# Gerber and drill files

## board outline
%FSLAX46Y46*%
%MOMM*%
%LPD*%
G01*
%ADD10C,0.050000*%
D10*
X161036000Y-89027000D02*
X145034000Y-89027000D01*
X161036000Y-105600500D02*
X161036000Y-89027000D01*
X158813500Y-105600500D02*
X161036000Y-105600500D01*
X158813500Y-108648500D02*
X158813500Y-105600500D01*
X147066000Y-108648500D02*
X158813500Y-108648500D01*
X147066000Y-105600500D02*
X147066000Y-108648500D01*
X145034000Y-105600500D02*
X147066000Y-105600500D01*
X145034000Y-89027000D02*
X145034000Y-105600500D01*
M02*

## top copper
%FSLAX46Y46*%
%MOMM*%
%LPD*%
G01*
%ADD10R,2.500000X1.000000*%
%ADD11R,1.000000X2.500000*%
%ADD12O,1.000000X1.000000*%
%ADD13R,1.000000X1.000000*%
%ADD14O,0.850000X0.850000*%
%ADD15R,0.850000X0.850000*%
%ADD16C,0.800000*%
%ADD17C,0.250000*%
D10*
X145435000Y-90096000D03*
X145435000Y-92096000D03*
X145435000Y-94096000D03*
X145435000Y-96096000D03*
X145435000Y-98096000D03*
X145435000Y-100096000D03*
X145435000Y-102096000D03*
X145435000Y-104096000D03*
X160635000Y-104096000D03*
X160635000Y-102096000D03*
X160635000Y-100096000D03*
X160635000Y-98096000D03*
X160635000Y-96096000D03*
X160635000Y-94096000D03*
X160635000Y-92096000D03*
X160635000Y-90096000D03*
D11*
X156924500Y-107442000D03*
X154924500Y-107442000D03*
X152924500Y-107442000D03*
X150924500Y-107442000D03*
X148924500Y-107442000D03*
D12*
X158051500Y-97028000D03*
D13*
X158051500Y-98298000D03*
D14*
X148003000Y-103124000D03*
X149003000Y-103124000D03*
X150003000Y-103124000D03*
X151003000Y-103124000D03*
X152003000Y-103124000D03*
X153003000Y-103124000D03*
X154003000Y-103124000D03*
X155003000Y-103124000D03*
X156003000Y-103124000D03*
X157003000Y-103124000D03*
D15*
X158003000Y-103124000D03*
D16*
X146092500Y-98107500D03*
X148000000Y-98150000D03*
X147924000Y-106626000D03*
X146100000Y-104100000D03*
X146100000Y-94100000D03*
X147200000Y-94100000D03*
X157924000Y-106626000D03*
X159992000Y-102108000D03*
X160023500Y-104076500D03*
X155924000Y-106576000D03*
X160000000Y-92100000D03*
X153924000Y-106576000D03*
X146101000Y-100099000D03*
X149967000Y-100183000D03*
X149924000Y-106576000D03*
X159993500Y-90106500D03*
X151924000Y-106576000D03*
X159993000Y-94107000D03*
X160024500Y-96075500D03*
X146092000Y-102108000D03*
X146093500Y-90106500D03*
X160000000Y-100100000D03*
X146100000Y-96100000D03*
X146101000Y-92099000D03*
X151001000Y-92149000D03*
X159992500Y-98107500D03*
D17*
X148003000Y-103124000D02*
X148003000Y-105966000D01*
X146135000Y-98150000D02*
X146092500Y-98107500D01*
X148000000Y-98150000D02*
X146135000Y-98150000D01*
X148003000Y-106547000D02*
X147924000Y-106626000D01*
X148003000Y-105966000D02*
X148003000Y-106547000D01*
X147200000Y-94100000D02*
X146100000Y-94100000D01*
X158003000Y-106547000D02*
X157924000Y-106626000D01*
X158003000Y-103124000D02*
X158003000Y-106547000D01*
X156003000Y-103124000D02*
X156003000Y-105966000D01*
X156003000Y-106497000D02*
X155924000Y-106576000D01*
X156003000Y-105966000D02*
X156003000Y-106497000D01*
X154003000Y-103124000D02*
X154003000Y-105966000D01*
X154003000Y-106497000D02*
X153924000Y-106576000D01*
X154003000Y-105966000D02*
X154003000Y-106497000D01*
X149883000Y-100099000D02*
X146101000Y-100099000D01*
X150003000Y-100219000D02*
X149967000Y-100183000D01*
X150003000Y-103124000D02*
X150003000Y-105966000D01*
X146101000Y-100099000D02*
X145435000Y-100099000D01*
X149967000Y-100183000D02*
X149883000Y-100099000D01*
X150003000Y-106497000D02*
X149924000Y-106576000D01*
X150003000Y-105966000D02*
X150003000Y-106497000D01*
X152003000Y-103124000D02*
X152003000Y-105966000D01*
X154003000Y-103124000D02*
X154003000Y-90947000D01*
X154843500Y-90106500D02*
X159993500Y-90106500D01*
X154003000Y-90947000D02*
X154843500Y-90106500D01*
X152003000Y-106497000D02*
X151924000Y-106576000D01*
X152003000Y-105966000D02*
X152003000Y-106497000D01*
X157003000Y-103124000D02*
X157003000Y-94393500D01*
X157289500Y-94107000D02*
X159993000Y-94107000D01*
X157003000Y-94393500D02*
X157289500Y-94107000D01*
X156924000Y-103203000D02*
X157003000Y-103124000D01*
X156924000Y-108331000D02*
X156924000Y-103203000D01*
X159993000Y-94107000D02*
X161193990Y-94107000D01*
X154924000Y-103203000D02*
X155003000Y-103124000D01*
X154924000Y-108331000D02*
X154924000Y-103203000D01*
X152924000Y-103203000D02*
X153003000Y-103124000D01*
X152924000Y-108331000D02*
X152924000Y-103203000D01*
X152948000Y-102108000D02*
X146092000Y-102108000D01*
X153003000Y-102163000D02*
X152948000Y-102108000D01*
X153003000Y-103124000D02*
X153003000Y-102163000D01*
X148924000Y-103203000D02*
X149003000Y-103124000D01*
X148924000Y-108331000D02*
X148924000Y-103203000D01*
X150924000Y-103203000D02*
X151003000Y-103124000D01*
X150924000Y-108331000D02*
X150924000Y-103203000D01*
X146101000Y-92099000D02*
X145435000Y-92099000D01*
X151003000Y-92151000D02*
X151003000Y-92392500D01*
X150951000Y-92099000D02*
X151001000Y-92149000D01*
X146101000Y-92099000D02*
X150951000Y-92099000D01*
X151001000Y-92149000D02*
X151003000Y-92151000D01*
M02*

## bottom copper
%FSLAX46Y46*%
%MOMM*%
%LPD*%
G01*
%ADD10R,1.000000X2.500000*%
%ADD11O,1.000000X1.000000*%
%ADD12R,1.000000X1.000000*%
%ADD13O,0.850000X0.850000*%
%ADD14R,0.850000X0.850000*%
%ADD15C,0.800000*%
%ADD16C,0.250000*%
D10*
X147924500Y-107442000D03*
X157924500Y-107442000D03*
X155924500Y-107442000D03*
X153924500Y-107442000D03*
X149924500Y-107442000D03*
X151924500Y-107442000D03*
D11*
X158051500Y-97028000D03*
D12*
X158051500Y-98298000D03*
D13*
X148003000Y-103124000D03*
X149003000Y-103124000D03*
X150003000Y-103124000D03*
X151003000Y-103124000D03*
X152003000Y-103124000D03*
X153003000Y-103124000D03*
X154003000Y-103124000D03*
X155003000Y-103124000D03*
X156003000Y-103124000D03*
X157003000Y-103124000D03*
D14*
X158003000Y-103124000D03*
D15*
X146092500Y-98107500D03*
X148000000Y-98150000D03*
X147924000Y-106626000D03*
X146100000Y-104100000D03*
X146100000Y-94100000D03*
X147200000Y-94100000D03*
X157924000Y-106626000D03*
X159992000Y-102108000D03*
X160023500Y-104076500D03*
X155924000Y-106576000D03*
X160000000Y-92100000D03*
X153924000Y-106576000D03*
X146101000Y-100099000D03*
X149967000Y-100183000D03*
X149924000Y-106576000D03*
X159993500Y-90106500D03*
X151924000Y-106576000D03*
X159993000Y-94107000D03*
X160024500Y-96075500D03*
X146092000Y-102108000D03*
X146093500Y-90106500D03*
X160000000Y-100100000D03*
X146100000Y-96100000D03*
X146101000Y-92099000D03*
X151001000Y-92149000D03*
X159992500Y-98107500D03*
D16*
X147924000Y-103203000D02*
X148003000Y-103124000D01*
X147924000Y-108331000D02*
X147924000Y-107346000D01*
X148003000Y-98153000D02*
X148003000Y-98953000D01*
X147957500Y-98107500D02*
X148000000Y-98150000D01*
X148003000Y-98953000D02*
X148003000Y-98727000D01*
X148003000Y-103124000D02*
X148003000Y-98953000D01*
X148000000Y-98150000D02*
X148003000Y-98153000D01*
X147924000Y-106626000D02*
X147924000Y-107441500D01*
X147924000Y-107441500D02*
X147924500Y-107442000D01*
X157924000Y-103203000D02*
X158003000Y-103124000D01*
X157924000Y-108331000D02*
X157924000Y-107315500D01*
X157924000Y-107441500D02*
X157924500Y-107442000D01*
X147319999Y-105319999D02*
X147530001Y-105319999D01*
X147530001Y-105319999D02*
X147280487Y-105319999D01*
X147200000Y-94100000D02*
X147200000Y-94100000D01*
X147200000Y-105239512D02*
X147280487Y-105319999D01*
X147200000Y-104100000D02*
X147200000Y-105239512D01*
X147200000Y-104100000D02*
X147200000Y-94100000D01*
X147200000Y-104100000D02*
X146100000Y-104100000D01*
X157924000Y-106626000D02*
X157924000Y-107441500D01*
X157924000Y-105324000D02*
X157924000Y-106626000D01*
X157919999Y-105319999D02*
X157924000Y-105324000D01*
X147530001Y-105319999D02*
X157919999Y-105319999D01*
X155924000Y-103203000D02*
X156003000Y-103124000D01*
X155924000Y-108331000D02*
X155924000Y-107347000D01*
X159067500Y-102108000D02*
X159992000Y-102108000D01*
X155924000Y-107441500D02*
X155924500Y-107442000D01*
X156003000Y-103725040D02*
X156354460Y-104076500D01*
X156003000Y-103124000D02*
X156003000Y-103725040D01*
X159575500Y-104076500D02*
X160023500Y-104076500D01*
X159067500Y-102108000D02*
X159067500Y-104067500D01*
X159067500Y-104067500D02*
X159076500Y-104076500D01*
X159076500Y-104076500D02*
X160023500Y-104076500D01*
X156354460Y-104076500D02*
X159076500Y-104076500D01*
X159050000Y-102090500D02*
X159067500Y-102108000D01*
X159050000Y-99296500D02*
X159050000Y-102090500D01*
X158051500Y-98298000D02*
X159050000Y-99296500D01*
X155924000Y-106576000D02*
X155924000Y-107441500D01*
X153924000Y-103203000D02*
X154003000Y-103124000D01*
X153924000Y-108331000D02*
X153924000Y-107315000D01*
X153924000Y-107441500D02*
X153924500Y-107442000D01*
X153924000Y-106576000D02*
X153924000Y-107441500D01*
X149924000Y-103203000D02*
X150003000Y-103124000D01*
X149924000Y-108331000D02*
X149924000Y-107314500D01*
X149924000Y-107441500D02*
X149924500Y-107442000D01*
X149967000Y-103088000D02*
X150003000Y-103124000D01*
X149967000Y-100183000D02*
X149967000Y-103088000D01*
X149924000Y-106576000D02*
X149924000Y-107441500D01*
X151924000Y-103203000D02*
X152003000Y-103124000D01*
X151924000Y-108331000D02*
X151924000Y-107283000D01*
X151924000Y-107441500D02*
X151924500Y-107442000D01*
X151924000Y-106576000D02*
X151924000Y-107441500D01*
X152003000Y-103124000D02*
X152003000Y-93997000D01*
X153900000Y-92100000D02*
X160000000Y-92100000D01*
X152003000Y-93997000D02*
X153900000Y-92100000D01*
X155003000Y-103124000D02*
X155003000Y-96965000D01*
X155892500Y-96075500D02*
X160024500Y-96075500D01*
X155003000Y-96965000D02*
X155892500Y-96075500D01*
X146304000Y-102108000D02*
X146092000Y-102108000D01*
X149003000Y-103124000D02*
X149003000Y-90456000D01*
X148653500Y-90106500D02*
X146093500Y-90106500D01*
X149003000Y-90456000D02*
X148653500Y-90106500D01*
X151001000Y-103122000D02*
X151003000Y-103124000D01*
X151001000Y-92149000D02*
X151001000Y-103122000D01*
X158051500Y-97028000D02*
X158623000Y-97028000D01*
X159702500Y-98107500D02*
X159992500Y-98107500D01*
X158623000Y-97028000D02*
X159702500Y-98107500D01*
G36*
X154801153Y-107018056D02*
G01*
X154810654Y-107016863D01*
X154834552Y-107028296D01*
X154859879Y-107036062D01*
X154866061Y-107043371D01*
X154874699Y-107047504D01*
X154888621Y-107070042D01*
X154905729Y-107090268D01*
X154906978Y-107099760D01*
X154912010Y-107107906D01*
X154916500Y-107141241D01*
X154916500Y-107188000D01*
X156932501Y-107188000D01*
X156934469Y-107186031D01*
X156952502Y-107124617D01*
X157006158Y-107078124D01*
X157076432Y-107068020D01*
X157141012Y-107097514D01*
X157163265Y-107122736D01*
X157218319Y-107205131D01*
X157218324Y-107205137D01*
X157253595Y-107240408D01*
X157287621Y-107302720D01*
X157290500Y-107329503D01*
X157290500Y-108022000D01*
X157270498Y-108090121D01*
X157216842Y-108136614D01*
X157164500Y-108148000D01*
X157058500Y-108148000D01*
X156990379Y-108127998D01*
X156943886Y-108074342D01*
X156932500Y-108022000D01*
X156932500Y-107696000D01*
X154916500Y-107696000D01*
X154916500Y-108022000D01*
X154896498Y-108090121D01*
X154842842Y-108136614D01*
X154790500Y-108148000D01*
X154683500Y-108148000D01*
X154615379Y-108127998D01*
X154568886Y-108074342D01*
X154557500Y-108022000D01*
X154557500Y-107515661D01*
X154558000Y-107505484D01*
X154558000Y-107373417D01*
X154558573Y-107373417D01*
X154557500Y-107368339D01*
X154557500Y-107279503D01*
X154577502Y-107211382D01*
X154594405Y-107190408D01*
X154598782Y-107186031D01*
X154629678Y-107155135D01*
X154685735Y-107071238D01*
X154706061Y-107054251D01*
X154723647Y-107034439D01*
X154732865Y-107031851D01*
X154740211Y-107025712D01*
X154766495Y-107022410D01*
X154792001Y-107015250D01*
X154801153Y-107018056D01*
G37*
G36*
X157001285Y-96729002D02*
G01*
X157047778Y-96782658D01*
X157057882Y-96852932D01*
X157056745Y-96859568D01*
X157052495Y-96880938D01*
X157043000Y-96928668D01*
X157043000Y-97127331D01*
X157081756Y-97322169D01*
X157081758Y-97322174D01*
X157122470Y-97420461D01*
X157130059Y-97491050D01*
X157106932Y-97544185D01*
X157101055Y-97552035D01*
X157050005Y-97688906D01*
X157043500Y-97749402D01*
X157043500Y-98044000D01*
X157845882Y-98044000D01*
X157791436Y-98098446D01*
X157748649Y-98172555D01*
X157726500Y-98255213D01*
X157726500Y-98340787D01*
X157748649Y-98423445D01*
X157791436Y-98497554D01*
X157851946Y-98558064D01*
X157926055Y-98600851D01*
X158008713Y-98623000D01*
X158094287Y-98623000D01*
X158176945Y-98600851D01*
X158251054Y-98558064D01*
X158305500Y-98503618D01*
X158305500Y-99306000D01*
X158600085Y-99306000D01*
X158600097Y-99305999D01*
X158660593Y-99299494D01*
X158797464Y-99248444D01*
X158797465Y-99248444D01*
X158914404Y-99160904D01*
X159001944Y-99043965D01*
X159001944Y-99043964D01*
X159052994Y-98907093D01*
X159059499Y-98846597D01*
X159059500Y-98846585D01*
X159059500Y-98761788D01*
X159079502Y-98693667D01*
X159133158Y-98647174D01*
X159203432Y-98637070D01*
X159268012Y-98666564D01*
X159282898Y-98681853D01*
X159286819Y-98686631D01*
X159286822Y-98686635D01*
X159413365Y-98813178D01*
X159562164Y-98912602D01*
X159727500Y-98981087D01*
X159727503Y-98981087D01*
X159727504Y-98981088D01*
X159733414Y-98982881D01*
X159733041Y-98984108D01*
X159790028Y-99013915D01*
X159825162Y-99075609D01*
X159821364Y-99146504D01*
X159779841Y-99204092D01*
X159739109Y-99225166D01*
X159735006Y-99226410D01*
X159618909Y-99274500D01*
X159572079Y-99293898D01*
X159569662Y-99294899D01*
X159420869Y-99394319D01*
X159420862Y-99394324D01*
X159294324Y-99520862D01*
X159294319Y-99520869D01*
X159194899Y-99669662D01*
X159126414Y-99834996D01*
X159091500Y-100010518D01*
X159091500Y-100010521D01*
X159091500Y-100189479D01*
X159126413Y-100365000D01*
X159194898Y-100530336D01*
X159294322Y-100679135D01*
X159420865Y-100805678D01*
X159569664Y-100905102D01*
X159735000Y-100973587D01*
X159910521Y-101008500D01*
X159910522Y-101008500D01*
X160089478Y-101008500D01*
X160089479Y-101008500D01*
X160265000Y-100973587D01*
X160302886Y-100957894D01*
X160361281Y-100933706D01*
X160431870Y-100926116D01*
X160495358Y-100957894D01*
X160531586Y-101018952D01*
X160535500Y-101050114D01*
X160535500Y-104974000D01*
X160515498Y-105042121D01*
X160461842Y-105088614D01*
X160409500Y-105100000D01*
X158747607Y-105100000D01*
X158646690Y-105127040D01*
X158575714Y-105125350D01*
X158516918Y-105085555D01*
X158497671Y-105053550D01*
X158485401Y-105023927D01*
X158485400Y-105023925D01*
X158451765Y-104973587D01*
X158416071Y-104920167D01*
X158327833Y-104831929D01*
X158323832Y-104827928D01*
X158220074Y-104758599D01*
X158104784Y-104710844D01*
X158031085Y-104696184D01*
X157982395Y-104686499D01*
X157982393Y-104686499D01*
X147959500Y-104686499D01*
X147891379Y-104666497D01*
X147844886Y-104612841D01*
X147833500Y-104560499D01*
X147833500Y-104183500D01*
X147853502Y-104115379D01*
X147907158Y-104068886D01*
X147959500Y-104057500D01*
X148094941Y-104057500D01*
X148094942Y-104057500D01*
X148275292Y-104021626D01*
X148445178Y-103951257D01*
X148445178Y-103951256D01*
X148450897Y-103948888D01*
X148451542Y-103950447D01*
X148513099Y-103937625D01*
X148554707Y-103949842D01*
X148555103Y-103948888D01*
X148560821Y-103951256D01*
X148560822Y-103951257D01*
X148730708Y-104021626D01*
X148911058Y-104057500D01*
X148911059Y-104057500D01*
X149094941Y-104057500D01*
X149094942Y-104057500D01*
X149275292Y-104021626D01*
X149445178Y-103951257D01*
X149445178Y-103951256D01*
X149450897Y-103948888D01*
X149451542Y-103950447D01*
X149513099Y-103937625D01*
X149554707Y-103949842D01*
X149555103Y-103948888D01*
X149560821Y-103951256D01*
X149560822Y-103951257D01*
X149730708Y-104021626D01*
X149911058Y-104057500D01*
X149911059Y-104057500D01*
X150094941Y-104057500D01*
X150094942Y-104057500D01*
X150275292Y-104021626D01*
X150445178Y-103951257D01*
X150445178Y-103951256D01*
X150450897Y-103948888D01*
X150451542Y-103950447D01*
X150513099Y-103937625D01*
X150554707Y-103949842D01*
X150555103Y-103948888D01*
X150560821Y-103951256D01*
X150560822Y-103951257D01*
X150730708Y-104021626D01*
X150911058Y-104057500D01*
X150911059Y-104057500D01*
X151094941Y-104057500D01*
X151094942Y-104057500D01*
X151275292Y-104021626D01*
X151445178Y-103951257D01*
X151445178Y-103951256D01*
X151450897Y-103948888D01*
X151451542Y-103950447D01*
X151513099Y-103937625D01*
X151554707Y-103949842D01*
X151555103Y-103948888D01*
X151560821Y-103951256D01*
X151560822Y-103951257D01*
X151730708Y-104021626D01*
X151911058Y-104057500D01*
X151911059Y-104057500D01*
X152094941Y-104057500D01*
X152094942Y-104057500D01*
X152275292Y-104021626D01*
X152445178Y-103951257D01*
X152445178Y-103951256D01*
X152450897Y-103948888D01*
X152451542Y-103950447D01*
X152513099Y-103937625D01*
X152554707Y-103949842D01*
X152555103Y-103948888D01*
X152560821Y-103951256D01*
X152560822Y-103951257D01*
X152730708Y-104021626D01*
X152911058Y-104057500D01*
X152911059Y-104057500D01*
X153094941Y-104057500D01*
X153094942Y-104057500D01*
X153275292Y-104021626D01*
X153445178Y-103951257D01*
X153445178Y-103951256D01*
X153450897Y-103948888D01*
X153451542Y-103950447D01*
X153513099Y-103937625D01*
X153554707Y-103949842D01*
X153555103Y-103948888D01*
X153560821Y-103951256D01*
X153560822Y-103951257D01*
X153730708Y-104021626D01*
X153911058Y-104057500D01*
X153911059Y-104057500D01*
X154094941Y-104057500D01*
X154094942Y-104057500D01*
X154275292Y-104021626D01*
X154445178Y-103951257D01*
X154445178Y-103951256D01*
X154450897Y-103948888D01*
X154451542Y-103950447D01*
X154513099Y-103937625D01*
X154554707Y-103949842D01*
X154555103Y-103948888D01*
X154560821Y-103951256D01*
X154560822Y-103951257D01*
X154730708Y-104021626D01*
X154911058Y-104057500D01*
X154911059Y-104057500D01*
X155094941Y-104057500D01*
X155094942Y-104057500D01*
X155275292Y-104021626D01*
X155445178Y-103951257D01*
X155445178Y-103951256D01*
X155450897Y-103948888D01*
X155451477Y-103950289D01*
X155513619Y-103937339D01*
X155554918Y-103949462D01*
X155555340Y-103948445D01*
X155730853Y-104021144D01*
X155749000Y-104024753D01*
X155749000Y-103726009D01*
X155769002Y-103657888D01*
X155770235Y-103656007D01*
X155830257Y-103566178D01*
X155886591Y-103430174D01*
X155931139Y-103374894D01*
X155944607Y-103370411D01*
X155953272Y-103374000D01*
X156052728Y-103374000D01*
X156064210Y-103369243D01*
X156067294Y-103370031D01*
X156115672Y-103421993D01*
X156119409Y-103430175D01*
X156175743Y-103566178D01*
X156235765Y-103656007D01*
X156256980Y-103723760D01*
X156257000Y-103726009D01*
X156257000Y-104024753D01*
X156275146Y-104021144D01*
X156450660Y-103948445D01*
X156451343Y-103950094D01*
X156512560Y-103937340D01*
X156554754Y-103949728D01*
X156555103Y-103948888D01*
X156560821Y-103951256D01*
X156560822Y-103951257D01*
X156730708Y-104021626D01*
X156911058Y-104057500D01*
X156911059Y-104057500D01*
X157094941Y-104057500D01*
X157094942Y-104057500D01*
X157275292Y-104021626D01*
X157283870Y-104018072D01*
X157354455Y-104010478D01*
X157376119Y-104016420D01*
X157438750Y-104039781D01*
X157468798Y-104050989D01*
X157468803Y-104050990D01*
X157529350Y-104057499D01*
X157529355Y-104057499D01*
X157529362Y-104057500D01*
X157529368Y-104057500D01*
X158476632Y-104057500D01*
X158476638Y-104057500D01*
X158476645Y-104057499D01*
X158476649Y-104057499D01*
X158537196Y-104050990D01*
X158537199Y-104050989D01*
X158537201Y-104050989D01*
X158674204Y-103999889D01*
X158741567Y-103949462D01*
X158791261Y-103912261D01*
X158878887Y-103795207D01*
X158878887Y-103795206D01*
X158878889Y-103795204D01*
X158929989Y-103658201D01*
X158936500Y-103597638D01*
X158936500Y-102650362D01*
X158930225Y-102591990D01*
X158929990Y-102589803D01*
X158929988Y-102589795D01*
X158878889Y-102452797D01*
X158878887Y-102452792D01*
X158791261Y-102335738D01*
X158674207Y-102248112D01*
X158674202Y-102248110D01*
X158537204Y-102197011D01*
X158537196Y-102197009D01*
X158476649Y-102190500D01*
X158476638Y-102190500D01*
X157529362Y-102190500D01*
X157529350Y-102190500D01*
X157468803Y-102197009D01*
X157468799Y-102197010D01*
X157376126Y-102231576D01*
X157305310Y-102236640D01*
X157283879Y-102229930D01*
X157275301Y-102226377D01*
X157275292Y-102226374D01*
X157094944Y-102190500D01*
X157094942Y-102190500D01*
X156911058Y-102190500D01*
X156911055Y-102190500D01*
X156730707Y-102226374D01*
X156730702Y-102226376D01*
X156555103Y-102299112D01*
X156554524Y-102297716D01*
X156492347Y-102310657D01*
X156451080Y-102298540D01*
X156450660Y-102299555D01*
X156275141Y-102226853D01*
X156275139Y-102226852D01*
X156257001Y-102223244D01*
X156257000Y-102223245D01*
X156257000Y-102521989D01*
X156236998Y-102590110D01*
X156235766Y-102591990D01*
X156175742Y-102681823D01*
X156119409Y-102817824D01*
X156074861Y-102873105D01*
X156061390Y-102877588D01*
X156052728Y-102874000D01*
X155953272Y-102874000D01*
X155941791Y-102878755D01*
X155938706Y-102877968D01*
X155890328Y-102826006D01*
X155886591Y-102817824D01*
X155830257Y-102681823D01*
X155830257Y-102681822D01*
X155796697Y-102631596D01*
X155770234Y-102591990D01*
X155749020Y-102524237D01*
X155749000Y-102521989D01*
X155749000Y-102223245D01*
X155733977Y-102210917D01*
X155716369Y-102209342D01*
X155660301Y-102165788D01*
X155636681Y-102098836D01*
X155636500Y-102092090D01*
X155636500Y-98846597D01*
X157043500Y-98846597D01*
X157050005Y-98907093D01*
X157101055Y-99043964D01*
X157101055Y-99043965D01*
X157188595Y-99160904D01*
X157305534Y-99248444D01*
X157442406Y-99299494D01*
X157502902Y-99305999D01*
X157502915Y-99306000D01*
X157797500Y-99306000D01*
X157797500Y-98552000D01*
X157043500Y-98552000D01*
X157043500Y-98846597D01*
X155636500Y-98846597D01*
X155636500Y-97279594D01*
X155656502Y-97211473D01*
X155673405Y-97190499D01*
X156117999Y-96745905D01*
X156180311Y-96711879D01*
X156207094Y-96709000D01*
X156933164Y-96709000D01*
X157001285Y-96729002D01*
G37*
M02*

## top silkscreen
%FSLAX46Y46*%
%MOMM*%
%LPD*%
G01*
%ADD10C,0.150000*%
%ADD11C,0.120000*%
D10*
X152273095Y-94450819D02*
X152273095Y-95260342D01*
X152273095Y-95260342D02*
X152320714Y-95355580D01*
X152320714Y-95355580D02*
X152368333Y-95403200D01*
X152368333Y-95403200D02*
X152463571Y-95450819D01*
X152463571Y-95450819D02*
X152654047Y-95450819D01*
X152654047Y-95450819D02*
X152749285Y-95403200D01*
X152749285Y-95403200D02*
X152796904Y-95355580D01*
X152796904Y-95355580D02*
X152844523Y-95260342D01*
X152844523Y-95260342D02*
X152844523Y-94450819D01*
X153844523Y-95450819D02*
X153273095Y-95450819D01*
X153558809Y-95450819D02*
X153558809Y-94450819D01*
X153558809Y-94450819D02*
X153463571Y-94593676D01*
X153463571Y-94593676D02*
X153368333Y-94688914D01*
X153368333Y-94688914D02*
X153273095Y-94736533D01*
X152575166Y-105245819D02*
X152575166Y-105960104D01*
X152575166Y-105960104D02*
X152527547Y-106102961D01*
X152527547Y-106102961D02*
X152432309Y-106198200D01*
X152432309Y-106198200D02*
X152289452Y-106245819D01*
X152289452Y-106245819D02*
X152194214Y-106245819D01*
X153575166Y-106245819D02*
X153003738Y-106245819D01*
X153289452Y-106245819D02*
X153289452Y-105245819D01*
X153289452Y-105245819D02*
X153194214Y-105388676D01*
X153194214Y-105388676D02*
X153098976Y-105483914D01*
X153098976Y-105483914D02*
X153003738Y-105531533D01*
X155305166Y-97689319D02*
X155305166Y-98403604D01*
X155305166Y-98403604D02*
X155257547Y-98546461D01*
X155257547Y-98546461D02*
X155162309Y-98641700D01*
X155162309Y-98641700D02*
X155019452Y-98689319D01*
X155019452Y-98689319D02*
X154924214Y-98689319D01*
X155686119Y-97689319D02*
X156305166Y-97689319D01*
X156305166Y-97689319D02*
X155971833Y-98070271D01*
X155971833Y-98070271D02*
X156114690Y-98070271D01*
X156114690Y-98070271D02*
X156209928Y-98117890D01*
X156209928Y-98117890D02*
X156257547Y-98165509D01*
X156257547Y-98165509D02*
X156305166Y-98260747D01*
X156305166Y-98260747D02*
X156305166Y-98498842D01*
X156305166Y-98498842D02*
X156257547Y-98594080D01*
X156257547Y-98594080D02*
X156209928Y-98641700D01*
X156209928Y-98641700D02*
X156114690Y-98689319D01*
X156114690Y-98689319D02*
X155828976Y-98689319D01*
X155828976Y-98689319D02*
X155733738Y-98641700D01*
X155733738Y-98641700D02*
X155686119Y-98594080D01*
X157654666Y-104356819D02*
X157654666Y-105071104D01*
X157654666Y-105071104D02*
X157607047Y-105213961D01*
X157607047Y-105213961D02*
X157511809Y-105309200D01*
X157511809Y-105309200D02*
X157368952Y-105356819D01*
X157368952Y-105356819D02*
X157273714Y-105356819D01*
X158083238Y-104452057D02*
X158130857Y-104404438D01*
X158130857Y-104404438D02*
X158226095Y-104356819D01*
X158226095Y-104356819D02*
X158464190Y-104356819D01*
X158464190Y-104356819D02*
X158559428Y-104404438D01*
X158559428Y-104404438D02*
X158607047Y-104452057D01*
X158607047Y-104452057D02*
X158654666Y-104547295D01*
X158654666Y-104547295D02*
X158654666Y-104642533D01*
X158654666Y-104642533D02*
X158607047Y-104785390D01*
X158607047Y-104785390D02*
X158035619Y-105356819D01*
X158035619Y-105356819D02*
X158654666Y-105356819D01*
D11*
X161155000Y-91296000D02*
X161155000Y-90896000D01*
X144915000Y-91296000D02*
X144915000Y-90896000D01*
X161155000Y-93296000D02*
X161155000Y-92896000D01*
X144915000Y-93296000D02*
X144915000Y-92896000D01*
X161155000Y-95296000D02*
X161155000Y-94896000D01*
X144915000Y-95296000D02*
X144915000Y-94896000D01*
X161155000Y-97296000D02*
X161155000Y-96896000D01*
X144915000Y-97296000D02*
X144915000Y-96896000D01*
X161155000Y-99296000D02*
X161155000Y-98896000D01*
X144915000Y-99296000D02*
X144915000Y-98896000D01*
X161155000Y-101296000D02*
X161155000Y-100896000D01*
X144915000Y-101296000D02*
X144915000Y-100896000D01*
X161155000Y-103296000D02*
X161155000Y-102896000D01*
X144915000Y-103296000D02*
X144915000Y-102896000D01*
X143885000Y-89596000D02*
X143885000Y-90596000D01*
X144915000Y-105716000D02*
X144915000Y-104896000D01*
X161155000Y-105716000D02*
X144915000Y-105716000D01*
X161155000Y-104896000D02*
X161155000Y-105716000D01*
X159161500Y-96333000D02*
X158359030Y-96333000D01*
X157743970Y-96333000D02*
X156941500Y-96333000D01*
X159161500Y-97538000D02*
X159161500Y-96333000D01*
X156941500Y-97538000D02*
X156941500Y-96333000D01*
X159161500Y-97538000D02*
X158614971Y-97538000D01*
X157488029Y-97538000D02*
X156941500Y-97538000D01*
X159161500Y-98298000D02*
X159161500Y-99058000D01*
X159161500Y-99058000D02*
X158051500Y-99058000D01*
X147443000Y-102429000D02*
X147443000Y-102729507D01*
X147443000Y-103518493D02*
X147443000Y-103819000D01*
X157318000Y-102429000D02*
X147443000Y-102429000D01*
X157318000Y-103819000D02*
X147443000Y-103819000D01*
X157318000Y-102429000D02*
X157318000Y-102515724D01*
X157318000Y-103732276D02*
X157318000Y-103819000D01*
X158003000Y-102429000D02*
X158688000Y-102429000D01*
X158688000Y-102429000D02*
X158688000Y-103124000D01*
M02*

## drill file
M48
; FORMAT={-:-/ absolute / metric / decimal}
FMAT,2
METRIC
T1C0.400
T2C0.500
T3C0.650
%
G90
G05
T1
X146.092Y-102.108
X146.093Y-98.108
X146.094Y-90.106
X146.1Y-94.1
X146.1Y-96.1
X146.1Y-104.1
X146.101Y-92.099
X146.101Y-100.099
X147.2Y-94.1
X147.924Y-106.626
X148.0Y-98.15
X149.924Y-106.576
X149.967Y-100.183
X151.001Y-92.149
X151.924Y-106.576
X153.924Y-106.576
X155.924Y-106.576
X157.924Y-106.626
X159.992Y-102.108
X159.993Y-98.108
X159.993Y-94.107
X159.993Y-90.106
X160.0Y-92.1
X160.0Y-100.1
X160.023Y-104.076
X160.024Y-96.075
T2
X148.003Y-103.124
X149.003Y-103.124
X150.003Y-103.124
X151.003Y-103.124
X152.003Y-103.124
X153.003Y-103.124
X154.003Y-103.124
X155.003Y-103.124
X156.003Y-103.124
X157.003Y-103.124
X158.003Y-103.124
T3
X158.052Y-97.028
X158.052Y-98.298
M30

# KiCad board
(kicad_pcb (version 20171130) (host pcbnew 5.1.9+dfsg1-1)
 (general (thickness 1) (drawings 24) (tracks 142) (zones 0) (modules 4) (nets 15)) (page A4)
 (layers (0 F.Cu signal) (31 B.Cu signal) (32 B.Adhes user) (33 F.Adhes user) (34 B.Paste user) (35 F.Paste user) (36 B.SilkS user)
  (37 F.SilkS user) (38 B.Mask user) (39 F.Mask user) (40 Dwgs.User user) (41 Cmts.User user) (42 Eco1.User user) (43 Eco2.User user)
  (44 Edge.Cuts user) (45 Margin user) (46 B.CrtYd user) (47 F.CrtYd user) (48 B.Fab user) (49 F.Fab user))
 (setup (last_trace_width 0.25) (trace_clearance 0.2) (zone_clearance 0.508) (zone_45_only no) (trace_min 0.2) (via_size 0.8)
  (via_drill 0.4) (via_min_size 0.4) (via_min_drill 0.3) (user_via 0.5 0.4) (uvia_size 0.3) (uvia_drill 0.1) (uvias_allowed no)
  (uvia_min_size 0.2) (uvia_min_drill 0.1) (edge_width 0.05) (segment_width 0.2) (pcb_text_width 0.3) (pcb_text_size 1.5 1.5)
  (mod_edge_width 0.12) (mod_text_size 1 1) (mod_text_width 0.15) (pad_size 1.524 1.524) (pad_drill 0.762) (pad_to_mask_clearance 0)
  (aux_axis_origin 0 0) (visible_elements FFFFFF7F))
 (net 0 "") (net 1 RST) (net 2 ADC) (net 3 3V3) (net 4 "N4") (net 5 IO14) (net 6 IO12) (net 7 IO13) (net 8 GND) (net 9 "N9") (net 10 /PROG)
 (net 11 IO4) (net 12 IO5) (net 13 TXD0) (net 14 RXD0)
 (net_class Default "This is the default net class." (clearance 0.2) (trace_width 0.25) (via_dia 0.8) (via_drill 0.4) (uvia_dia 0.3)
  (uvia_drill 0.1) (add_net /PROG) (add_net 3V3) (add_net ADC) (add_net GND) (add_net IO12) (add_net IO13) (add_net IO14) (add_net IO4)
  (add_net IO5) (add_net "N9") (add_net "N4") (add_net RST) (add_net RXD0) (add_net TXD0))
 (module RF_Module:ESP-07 (layer F.Cu) (at 153.035 94.996)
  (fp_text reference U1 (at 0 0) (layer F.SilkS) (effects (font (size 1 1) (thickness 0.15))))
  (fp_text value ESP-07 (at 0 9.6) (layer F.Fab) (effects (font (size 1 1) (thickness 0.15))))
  (fp_line (start 8.12 -3.7) (end 8.12 -4.1) (layer F.SilkS) (width 0.12))
  (fp_line (start -8.12 -3.7) (end -8.12 -4.1) (layer F.SilkS) (width 0.12))
  (fp_line (start 8.12 -1.7) (end 8.12 -2.1) (layer F.SilkS) (width 0.12))
  (fp_line (start -8.12 -1.7) (end -8.12 -2.1) (layer F.SilkS) (width 0.12))
  (fp_line (start 8.12 0.3) (end 8.12 -0.1) (layer F.SilkS) (width 0.12))
  (fp_line (start -8.12 0.3) (end -8.12 -0.1) (layer F.SilkS) (width 0.12))
  (fp_line (start 8.12 2.3) (end 8.12 1.9) (layer F.SilkS) (width 0.12))
  (fp_line (start -8.12 2.3) (end -8.12 1.9) (layer F.SilkS) (width 0.12))
  (fp_line (start 8.12 4.3) (end 8.12 3.9) (layer F.SilkS) (width 0.12))
  (fp_line (start -8.12 4.3) (end -8.12 3.9) (layer F.SilkS) (width 0.12))
  (fp_line (start 8.12 6.3) (end 8.12 5.9) (layer F.SilkS) (width 0.12))
  (fp_line (start -8.12 6.3) (end -8.12 5.9) (layer F.SilkS) (width 0.12))
  (fp_line (start 8.12 8.3) (end 8.12 7.9) (layer F.SilkS) (width 0.12))
  (fp_line (start -8.12 8.3) (end -8.12 7.9) (layer F.SilkS) (width 0.12))
  (fp_line (start -9.15 -5.4) (end -9.15 -4.4) (layer F.SilkS) (width 0.12))
  (fp_line (start -8.12 10.72) (end -8.12 9.9) (layer F.SilkS) (width 0.12))
  (fp_line (start 8.12 10.72) (end -8.12 10.72) (layer F.SilkS) (width 0.12))
  (fp_line (start 8.12 9.9) (end 8.12 10.72) (layer F.SilkS) (width 0.12))
  (pad 1 smd rect (at -7.6 -4.9) (size 2.5 1) (layers F.Cu F.Paste F.Mask) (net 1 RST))
  (pad 2 smd rect (at -7.6 -2.9) (size 2.5 1) (layers F.Cu F.Paste F.Mask) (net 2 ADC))
  (pad 3 smd rect (at -7.6 -0.9) (size 2.5 1) (layers F.Cu F.Paste F.Mask) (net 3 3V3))
  (pad 4 smd rect (at -7.6 1.1) (size 2.5 1) (layers F.Cu F.Paste F.Mask) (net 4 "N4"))
  (pad 5 smd rect (at -7.6 3.1) (size 2.5 1) (layers F.Cu F.Paste F.Mask) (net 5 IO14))
  (pad 6 smd rect (at -7.6 5.1) (size 2.5 1) (layers F.Cu F.Paste F.Mask) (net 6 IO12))
  (pad 7 smd rect (at -7.6 7.1) (size 2.5 1) (layers F.Cu F.Paste F.Mask) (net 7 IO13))
  (pad 8 smd rect (at -7.6 9.1) (size 2.5 1) (layers F.Cu F.Paste F.Mask) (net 3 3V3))
  (pad 9 smd rect (at 7.6 9.1) (size 2.5 1) (layers F.Cu F.Paste F.Mask) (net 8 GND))
  (pad 10 smd rect (at 7.6 7.1) (size 2.5 1) (layers F.Cu F.Paste F.Mask) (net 8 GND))
  (pad 11 smd rect (at 7.6 5.1) (size 2.5 1) (layers F.Cu F.Paste F.Mask) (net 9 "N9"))
  (pad 12 smd rect (at 7.6 3.1) (size 2.5 1) (layers F.Cu F.Paste F.Mask) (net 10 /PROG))
  (pad 13 smd rect (at 7.6 1.1) (size 2.5 1) (layers F.Cu F.Paste F.Mask) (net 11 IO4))
  (pad 14 smd rect (at 7.6 -0.9) (size 2.5 1) (layers F.Cu F.Paste F.Mask) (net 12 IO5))
  (pad 15 smd rect (at 7.6 -2.9) (size 2.5 1) (layers F.Cu F.Paste F.Mask) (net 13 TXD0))
  (pad 16 smd rect (at 7.6 -4.9) (size 2.5 1) (layers F.Cu F.Paste F.Mask) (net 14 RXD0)))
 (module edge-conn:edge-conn (layer F.Cu) (at 152.9245 107.442)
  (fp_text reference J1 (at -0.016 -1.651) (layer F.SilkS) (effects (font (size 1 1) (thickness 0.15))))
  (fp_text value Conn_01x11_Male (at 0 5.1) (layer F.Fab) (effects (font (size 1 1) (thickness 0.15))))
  (pad 11 connect rect (at -5 0) (size 1 2.5) (layers B.Cu B.Mask) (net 5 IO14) (clearance 0.01))
  (pad 1 connect rect (at 5 0) (size 1 2.5) (layers B.Cu B.Mask) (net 3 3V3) (clearance 0.01))
  (pad 3 connect rect (at 3 0) (size 1 2.5) (layers B.Cu B.Mask) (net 8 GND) (clearance 0.01))
  (pad 5 connect rect (at 1 0) (size 1 2.5) (layers B.Cu B.Mask) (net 14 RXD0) (clearance 0.01))
  (pad 9 connect rect (at -3 0) (size 1 2.5) (layers B.Cu B.Mask) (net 6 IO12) (clearance 0.01))
  (pad 7 connect rect (at -1 0) (size 1 2.5) (layers B.Cu B.Mask) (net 13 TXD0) (clearance 0.01))
  (pad 2 connect rect (at 4 0) (size 1 2.5) (layers F.Cu F.Mask) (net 12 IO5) (clearance 0.01))
  (pad 4 connect rect (at 2 0) (size 1 2.5) (layers F.Cu F.Mask) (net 11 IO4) (clearance 0.01))
  (pad 6 connect rect (at 0 0) (size 1 2.5) (layers F.Cu F.Mask) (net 7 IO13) (clearance 0.01))
  (pad 8 connect rect (at -2 0) (size 1 2.5) (layers F.Cu F.Mask) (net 2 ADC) (clearance 0.01))
  (pad 10 connect rect (at -4 0) (size 1 2.5) (layers F.Cu F.Mask) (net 1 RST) (clearance 0.01)))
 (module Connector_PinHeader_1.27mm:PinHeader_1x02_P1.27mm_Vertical (layer F.Cu) (at 158.0515 98.298 180)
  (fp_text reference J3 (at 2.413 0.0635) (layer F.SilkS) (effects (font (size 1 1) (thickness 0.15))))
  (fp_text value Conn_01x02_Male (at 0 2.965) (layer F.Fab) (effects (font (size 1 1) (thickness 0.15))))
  (fp_line (start -1.11 1.965) (end -0.30753 1.965) (layer F.SilkS) (width 0.12))
  (fp_line (start 0.30753 1.965) (end 1.11 1.965) (layer F.SilkS) (width 0.12))
  (fp_line (start -1.11 0.76) (end -1.11 1.965) (layer F.SilkS) (width 0.12))
  (fp_line (start 1.11 0.76) (end 1.11 1.965) (layer F.SilkS) (width 0.12))
  (fp_line (start -1.11 0.76) (end -0.563471 0.76) (layer F.SilkS) (width 0.12))
  (fp_line (start 0.563471 0.76) (end 1.11 0.76) (layer F.SilkS) (width 0.12))
  (fp_line (start -1.11 0) (end -1.11 -0.76) (layer F.SilkS) (width 0.12))
  (fp_line (start -1.11 -0.76) (end 0 -0.76) (layer F.SilkS) (width 0.12))
  (pad 2 thru_hole oval (at 0 1.27 180) (size 1 1) (drill 0.65) (layers *.Cu *.Mask) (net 10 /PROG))
  (pad 1 thru_hole rect (at 0 0 180) (size 1 1) (drill 0.65) (layers *.Cu *.Mask) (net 8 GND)))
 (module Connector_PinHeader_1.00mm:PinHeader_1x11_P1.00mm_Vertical (layer F.Cu) (at 158.003 103.124 270)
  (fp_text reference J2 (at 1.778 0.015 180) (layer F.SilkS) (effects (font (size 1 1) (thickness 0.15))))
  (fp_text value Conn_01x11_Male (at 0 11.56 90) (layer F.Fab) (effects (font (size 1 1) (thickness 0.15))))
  (fp_line (start -0.695 10.56) (end -0.394493 10.56) (layer F.SilkS) (width 0.12))
  (fp_line (start 0.394493 10.56) (end 0.695 10.56) (layer F.SilkS) (width 0.12))
  (fp_line (start -0.695 0.685) (end -0.695 10.56) (layer F.SilkS) (width 0.12))
  (fp_line (start 0.695 0.685) (end 0.695 10.56) (layer F.SilkS) (width 0.12))
  (fp_line (start -0.695 0.685) (end -0.608276 0.685) (layer F.SilkS) (width 0.12))
  (fp_line (start 0.608276 0.685) (end 0.695 0.685) (layer F.SilkS) (width 0.12))
  (fp_line (start -0.695 0) (end -0.695 -0.685) (layer F.SilkS) (width 0.12))
  (fp_line (start -0.695 -0.685) (end 0 -0.685) (layer F.SilkS) (width 0.12))
  (pad 11 thru_hole oval (at 0 10 270) (size 0.85 0.85) (drill 0.5) (layers *.Cu *.Mask) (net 5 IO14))
  (pad 10 thru_hole oval (at 0 9 270) (size 0.85 0.85) (drill 0.5) (layers *.Cu *.Mask) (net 1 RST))
  (pad 9 thru_hole oval (at 0 8 270) (size 0.85 0.85) (drill 0.5) (layers *.Cu *.Mask) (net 6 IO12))
  (pad 8 thru_hole oval (at 0 7 270) (size 0.85 0.85) (drill 0.5) (layers *.Cu *.Mask) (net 2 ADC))
  (pad 7 thru_hole oval (at 0 6 270) (size 0.85 0.85) (drill 0.5) (layers *.Cu *.Mask) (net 13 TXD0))
  (pad 6 thru_hole oval (at 0 5 270) (size 0.85 0.85) (drill 0.5) (layers *.Cu *.Mask) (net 7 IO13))
  (pad 5 thru_hole oval (at 0 4 270) (size 0.85 0.85) (drill 0.5) (layers *.Cu *.Mask) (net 14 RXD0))
  (pad 4 thru_hole oval (at 0 3 270) (size 0.85 0.85) (drill 0.5) (layers *.Cu *.Mask) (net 11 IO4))
  (pad 3 thru_hole oval (at 0 2 270) (size 0.85 0.85) (drill 0.5) (layers *.Cu *.Mask) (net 8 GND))
  (pad 2 thru_hole oval (at 0 1 270) (size 0.85 0.85) (drill 0.5) (layers *.Cu *.Mask) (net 12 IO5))
  (pad 1 thru_hole rect (at 0 0 270) (size 0.85 0.85) (drill 0.5) (layers *.Cu *.Mask) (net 3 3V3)))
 (gr_line (start 161.036 89.027) (end 145.034 89.027) (layer Edge.Cuts) (width 0.05))
 (gr_line (start 161.036 105.6005) (end 161.036 89.027) (layer Edge.Cuts) (width 0.05))
 (gr_line (start 158.8135 105.6005) (end 161.036 105.6005) (layer Edge.Cuts) (width 0.05))
 (gr_line (start 158.8135 108.6485) (end 158.8135 105.6005) (layer Edge.Cuts) (width 0.05))
 (gr_line (start 147.066 108.6485) (end 158.8135 108.6485) (layer Edge.Cuts) (width 0.05))
 (gr_line (start 147.066 105.6005) (end 147.066 108.6485) (layer Edge.Cuts) (width 0.05))
 (gr_line (start 145.034 105.6005) (end 147.066 105.6005) (layer Edge.Cuts) (width 0.05))
 (gr_line (start 145.034 89.027) (end 145.034 105.6005) (layer Edge.Cuts) (width 0.05))
 (segment (start 147.924 103.203) (end 148.003 103.124) (width 0.25) (layer B.Cu) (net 5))
 (segment (start 147.924 108.331) (end 147.924 107.346) (width 0.25) (layer B.Cu) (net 5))
 (segment (start 148.003 103.124) (end 148.003 105.966) (width 0.25) (layer F.Cu) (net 5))
 (via (at 146.0925 98.1075) (size 0.8) (drill 0.4) (layers F.Cu B.Cu) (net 5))
 (segment (start 148.003 98.153) (end 148.003 98.953) (width 0.25) (layer B.Cu) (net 5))
 (segment (start 147.9575 98.1075) (end 148 98.15) (width 0.25) (layer B.Cu) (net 5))
 (segment (start 148.003 98.953) (end 148.003 98.727) (width 0.25) (layer B.Cu) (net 5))
 (segment (start 148.003 103.124) (end 148.003 98.953) (width 0.25) (layer B.Cu) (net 5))
 (segment (start 148 98.15) (end 148.003 98.153) (width 0.25) (layer B.Cu) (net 5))
 (via (at 148 98.15) (size 0.8) (drill 0.4) (layers F.Cu B.Cu) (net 5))
 (segment (start 146.135 98.15) (end 146.0925 98.1075) (width 0.25) (layer F.Cu) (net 5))
 (segment (start 148 98.15) (end 146.135 98.15) (width 0.25) (layer F.Cu) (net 5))
 (segment (start 147.924 106.626) (end 147.924 107.4415) (width 0.25) (layer B.Cu) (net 5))
 (segment (start 147.924 107.4415) (end 147.9245 107.442) (width 0.25) (layer B.Cu) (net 5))
 (via (at 147.924 106.626) (size 0.8) (drill 0.4) (layers F.Cu B.Cu) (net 5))
 (segment (start 148.003 106.547) (end 147.924 106.626) (width 0.25) (layer F.Cu) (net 5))
 (segment (start 148.003 105.966) (end 148.003 106.547) (width 0.25) (layer F.Cu) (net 5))
 (via (at 146.1 104.1) (size 0.8) (drill 0.4) (layers F.Cu B.Cu) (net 3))
 (via (at 146.1 94.1) (size 0.8) (drill 0.4) (layers F.Cu B.Cu) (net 3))
 (segment (start 157.924 103.203) (end 158.003 103.124) (width 0.25) (layer B.Cu) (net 3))
 (segment (start 157.924 108.331) (end 157.924 107.3155) (width 0.25) (layer B.Cu) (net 3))
 (segment (start 157.924 107.4415) (end 157.9245 107.442) (width 0.25) (layer B.Cu) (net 3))
 (segment (start 147.319999 105.319999) (end 147.530001 105.319999) (width 0.25) (layer B.Cu) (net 3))
 (segment (start 147.530001 105.319999) (end 147.280487 105.319999) (width 0.25) (layer B.Cu) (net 3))
 (segment (start 147.2 94.1) (end 147.2 94.1) (width 0.25) (layer B.Cu) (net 3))
 (via (at 147.2 94.1) (size 0.8) (drill 0.4) (layers F.Cu B.Cu) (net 3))
 (segment (start 147.2 105.239512) (end 147.280487 105.319999) (width 0.25) (layer B.Cu) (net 3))
 (segment (start 147.2 104.1) (end 147.2 105.239512) (width 0.25) (layer B.Cu) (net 3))
 (segment (start 147.2 104.1) (end 147.2 94.1) (width 0.25) (layer B.Cu) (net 3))
 (segment (start 147.2 94.1) (end 146.1 94.1) (width 0.25) (layer F.Cu) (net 3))
 (segment (start 147.2 104.1) (end 146.1 104.1) (width 0.25) (layer B.Cu) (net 3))
 (segment (start 157.924 106.626) (end 157.924 107.4415) (width 0.25) (layer B.Cu) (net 3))
 (via (at 157.924 106.626) (size 0.8) (drill 0.4) (layers F.Cu B.Cu) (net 3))
 (segment (start 158.003 106.547) (end 157.924 106.626) (width 0.25) (layer F.Cu) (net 3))
 (segment (start 158.003 103.124) (end 158.003 106.547) (width 0.25) (layer F.Cu) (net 3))
 (segment (start 157.924 105.324) (end 157.924 106.626) (width 0.25) (layer B.Cu) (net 3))
 (segment (start 157.919999 105.319999) (end 157.924 105.324) (width 0.25) (layer B.Cu) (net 3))
 (segment (start 147.530001 105.319999) (end 157.919999 105.319999) (width 0.25) (layer B.Cu) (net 3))
 (segment (start 155.924 103.203) (end 156.003 103.124) (width 0.25) (layer B.Cu) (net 8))
 (segment (start 155.924 108.331) (end 155.924 107.347) (width 0.25) (layer B.Cu) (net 8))
 (segment (start 159.0675 102.108) (end 159.992 102.108) (width 0.25) (layer B.Cu) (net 8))
 (segment (start 156.003 103.124) (end 156.003 105.966) (width 0.25) (layer F.Cu) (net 8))
 (segment (start 155.924 107.4415) (end 155.9245 107.442) (width 0.25) (layer B.Cu) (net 8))
 (via (at 159.992 102.108) (size 0.8) (drill 0.4) (layers F.Cu B.Cu) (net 8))
 (segment (start 156.003 103.72504) (end 156.35446 104.0765) (width 0.25) (layer B.Cu) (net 8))
 (segment (start 156.003 103.124) (end 156.003 103.72504) (width 0.25) (layer B.Cu) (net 8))
 (via (at 160.0235 104.0765) (size 0.8) (drill 0.4) (layers F.Cu B.Cu) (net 8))
 (segment (start 159.5755 104.0765) (end 160.0235 104.0765) (width 0.25) (layer B.Cu) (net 8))
 (segment (start 159.0675 102.108) (end 159.0675 104.0675) (width 0.25) (layer B.Cu) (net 8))
 (segment (start 159.0675 104.0675) (end 159.0765 104.0765) (width 0.25) (layer B.Cu) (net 8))
 (segment (start 159.0765 104.0765) (end 160.0235 104.0765) (width 0.25) (layer B.Cu) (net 8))
 (segment (start 156.35446 104.0765) (end 159.0765 104.0765) (width 0.25) (layer B.Cu) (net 8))
 (segment (start 159.05 102.0905) (end 159.0675 102.108) (width 0.25) (layer B.Cu) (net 8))
 (segment (start 159.05 99.2965) (end 159.05 102.0905) (width 0.25) (layer B.Cu) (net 8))
 (segment (start 158.0515 98.298) (end 159.05 99.2965) (width 0.25) (layer B.Cu) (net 8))
 (segment (start 155.924 106.576) (end 155.924 107.4415) (width 0.25) (layer B.Cu) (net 8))
 (via (at 155.924 106.576) (size 0.8) (drill 0.4) (layers F.Cu B.Cu) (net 8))
 (segment (start 156.003 106.497) (end 155.924 106.576) (width 0.25) (layer F.Cu) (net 8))
 (segment (start 156.003 105.966) (end 156.003 106.497) (width 0.25) (layer F.Cu) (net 8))
 (via (at 160 92.1) (size 0.8) (drill 0.4) (layers F.Cu B.Cu) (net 13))
 (segment (start 153.924 103.203) (end 154.003 103.124) (width 0.25) (layer B.Cu) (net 14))
 (segment (start 153.924 108.331) (end 153.924 107.315) (width 0.25) (layer B.Cu) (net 14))
 (segment (start 154.003 103.124) (end 154.003 105.966) (width 0.25) (layer F.Cu) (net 14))
 (segment (start 153.924 107.4415) (end 153.9245 107.442) (width 0.25) (layer B.Cu) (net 14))
 (segment (start 153.924 106.576) (end 153.924 107.4415) (width 0.25) (layer B.Cu) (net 14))
 (via (at 153.924 106.576) (size 0.8) (drill 0.4) (layers F.Cu B.Cu) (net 14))
 (segment (start 154.003 106.497) (end 153.924 106.576) (width 0.25) (layer F.Cu) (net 14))
 (segment (start 154.003 105.966) (end 154.003 106.497) (width 0.25) (layer F.Cu) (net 14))
 (segment (start 149.883 100.099) (end 146.101 100.099) (width 0.25) (layer F.Cu) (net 6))
 (segment (start 150.003 100.219) (end 149.967 100.183) (width 0.25) (layer F.Cu) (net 6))
 (segment (start 149.924 103.203) (end 150.003 103.124) (width 0.25) (layer B.Cu) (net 6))
 (segment (start 149.924 108.331) (end 149.924 107.3145) (width 0.25) (layer B.Cu) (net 6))
 (segment (start 150.003 103.124) (end 150.003 105.966) (width 0.25) (layer F.Cu) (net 6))
 (segment (start 149.924 107.4415) (end 149.9245 107.442) (width 0.25) (layer B.Cu) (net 6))
 (segment (start 146.101 100.099) (end 145.435 100.099) (width 0.25) (layer F.Cu) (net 6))
 (via (at 146.101 100.099) (size 0.8) (drill 0.4) (layers F.Cu B.Cu) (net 6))
 (segment (start 149.967 100.183) (end 149.883 100.099) (width 0.25) (layer F.Cu) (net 6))
 (via (at 149.967 100.183) (size 0.8) (drill 0.4) (layers F.Cu B.Cu) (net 6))
 (segment (start 149.967 103.088) (end 150.003 103.124) (width 0.25) (layer B.Cu) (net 6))
 (segment (start 149.967 100.183) (end 149.967 103.088) (width 0.25) (layer B.Cu) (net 6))
 (segment (start 149.924 106.576) (end 149.924 107.4415) (width 0.25) (layer B.Cu) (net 6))
 (via (at 149.924 106.576) (size 0.8) (drill 0.4) (layers F.Cu B.Cu) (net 6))
 (segment (start 150.003 106.497) (end 149.924 106.576) (width 0.25) (layer F.Cu) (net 6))
 (segment (start 150.003 105.966) (end 150.003 106.497) (width 0.25) (layer F.Cu) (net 6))
 (segment (start 151.924 103.203) (end 152.003 103.124) (width 0.25) (layer B.Cu) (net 13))
 (segment (start 151.924 108.331) (end 151.924 107.283) (width 0.25) (layer B.Cu) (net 13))
 (segment (start 152.003 103.124) (end 152.003 105.966) (width 0.25) (layer F.Cu) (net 13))
 (segment (start 151.924 107.4415) (end 151.9245 107.442) (width 0.25) (layer B.Cu) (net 13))
 (via (at 159.9935 90.1065) (size 0.8) (drill 0.4) (layers F.Cu B.Cu) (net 14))
 (segment (start 154.003 103.124) (end 154.003 90.947) (width 0.25) (layer F.Cu) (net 14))
 (segment (start 154.8435 90.1065) (end 159.9935 90.1065) (width 0.25) (layer F.Cu) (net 14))
 (segment (start 154.003 90.947) (end 154.8435 90.1065) (width 0.25) (layer F.Cu) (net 14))
 (segment (start 151.924 106.576) (end 151.924 107.4415) (width 0.25) (layer B.Cu) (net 13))
 (via (at 151.924 106.576) (size 0.8) (drill 0.4) (layers F.Cu B.Cu) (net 13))
 (segment (start 152.003 106.497) (end 151.924 106.576) (width 0.25) (layer F.Cu) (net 13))
 (segment (start 152.003 105.966) (end 152.003 106.497) (width 0.25) (layer F.Cu) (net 13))
 (segment (start 152.003 103.124) (end 152.003 93.997) (width 0.25) (layer B.Cu) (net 13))
 (segment (start 153.9 92.1) (end 160 92.1) (width 0.25) (layer B.Cu) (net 13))
 (segment (start 152.003 93.997) (end 153.9 92.1) (width 0.25) (layer B.Cu) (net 13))
 (segment (start 157.003 103.124) (end 157.003 94.3935) (width 0.25) (layer F.Cu) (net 12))
 (segment (start 157.2895 94.107) (end 159.993 94.107) (width 0.25) (layer F.Cu) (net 12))
 (segment (start 157.003 94.3935) (end 157.2895 94.107) (width 0.25) (layer F.Cu) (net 12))
 (segment (start 156.924 103.203) (end 157.003 103.124) (width 0.25) (layer F.Cu) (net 12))
 (segment (start 156.924 108.331) (end 156.924 103.203) (width 0.25) (layer F.Cu) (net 12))
 (segment (start 159.993 94.107) (end 161.19399 94.107) (width 0.25) (layer F.Cu) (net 12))
 (via (at 159.993 94.107) (size 0.8) (drill 0.4) (layers F.Cu B.Cu) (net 12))
 (segment (start 155.003 103.124) (end 155.003 96.965) (width 0.25) (layer B.Cu) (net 11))
 (segment (start 155.8925 96.0755) (end 160.0245 96.0755) (width 0.25) (layer B.Cu) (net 11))
 (segment (start 155.003 96.965) (end 155.8925 96.0755) (width 0.25) (layer B.Cu) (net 11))
 (segment (start 154.924 103.203) (end 155.003 103.124) (width 0.25) (layer F.Cu) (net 11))
 (segment (start 154.924 108.331) (end 154.924 103.203) (width 0.25) (layer F.Cu) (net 11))
 (via (at 160.0245 96.0755) (size 0.8) (drill 0.4) (layers F.Cu B.Cu) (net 11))
 (segment (start 152.924 103.203) (end 153.003 103.124) (width 0.25) (layer F.Cu) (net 7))
 (segment (start 152.924 108.331) (end 152.924 103.203) (width 0.25) (layer F.Cu) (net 7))
 (segment (start 146.304 102.108) (end 146.092 102.108) (width 0.25) (layer B.Cu) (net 7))
 (via (at 146.092 102.108) (size 0.8) (drill 0.4) (layers F.Cu B.Cu) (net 7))
 (segment (start 152.948 102.108) (end 146.092 102.108) (width 0.25) (layer F.Cu) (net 7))
 (segment (start 153.003 102.163) (end 152.948 102.108) (width 0.25) (layer F.Cu) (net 7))
 (segment (start 153.003 103.124) (end 153.003 102.163) (width 0.25) (layer F.Cu) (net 7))
 (segment (start 149.003 103.124) (end 149.003 90.456) (width 0.25) (layer B.Cu) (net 1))
 (segment (start 148.6535 90.1065) (end 146.0935 90.1065) (width 0.25) (layer B.Cu) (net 1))
 (segment (start 149.003 90.456) (end 148.6535 90.1065) (width 0.25) (layer B.Cu) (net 1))
 (segment (start 148.924 103.203) (end 149.003 103.124) (width 0.25) (layer F.Cu) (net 1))
 (segment (start 148.924 108.331) (end 148.924 103.203) (width 0.25) (layer F.Cu) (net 1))
 (via (at 146.0935 90.1065) (size 0.8) (drill 0.4) (layers F.Cu B.Cu) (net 1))
 (via (at 160 100.1) (size 0.8) (drill 0.4) (layers F.Cu B.Cu) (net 9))
 (via (at 146.1 96.1) (size 0.8) (drill 0.4) (layers F.Cu B.Cu) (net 4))
 (segment (start 150.924 103.203) (end 151.003 103.124) (width 0.25) (layer F.Cu) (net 2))
 (segment (start 150.924 108.331) (end 150.924 103.203) (width 0.25) (layer F.Cu) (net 2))
 (segment (start 146.101 92.099) (end 145.435 92.099) (width 0.25) (layer F.Cu) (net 2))
 (via (at 146.101 92.099) (size 0.8) (drill 0.4) (layers F.Cu B.Cu) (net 2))
 (segment (start 151.003 92.151) (end 151.003 92.3925) (width 0.25) (layer F.Cu) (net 2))
 (segment (start 150.951 92.099) (end 151.001 92.149) (width 0.25) (layer F.Cu) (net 2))
 (segment (start 146.101 92.099) (end 150.951 92.099) (width 0.25) (layer F.Cu) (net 2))
 (segment (start 151.001 92.149) (end 151.003 92.151) (width 0.25) (layer F.Cu) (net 2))
 (via (at 151.001 92.149) (size 0.8) (drill 0.4) (layers F.Cu B.Cu) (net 2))
 (segment (start 151.001 103.122) (end 151.003 103.124) (width 0.25) (layer B.Cu) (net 2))
 (segment (start 151.001 92.149) (end 151.001 103.122) (width 0.25) (layer B.Cu) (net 2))
 (segment (start 158.0515 97.028) (end 158.623 97.028) (width 0.25) (layer B.Cu) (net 10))
 (segment (start 159.7025 98.1075) (end 159.9925 98.1075) (width 0.25) (layer B.Cu) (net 10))
 (segment (start 158.623 97.028) (end 159.7025 98.1075) (width 0.25) (layer B.Cu) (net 10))
 (via (at 159.9925 98.1075) (size 0.8) (drill 0.4) (layers F.Cu B.Cu) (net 10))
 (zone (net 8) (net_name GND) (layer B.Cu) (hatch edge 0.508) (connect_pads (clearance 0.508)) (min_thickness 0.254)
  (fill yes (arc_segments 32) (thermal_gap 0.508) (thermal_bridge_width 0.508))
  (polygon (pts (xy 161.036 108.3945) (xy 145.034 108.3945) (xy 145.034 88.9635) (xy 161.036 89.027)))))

